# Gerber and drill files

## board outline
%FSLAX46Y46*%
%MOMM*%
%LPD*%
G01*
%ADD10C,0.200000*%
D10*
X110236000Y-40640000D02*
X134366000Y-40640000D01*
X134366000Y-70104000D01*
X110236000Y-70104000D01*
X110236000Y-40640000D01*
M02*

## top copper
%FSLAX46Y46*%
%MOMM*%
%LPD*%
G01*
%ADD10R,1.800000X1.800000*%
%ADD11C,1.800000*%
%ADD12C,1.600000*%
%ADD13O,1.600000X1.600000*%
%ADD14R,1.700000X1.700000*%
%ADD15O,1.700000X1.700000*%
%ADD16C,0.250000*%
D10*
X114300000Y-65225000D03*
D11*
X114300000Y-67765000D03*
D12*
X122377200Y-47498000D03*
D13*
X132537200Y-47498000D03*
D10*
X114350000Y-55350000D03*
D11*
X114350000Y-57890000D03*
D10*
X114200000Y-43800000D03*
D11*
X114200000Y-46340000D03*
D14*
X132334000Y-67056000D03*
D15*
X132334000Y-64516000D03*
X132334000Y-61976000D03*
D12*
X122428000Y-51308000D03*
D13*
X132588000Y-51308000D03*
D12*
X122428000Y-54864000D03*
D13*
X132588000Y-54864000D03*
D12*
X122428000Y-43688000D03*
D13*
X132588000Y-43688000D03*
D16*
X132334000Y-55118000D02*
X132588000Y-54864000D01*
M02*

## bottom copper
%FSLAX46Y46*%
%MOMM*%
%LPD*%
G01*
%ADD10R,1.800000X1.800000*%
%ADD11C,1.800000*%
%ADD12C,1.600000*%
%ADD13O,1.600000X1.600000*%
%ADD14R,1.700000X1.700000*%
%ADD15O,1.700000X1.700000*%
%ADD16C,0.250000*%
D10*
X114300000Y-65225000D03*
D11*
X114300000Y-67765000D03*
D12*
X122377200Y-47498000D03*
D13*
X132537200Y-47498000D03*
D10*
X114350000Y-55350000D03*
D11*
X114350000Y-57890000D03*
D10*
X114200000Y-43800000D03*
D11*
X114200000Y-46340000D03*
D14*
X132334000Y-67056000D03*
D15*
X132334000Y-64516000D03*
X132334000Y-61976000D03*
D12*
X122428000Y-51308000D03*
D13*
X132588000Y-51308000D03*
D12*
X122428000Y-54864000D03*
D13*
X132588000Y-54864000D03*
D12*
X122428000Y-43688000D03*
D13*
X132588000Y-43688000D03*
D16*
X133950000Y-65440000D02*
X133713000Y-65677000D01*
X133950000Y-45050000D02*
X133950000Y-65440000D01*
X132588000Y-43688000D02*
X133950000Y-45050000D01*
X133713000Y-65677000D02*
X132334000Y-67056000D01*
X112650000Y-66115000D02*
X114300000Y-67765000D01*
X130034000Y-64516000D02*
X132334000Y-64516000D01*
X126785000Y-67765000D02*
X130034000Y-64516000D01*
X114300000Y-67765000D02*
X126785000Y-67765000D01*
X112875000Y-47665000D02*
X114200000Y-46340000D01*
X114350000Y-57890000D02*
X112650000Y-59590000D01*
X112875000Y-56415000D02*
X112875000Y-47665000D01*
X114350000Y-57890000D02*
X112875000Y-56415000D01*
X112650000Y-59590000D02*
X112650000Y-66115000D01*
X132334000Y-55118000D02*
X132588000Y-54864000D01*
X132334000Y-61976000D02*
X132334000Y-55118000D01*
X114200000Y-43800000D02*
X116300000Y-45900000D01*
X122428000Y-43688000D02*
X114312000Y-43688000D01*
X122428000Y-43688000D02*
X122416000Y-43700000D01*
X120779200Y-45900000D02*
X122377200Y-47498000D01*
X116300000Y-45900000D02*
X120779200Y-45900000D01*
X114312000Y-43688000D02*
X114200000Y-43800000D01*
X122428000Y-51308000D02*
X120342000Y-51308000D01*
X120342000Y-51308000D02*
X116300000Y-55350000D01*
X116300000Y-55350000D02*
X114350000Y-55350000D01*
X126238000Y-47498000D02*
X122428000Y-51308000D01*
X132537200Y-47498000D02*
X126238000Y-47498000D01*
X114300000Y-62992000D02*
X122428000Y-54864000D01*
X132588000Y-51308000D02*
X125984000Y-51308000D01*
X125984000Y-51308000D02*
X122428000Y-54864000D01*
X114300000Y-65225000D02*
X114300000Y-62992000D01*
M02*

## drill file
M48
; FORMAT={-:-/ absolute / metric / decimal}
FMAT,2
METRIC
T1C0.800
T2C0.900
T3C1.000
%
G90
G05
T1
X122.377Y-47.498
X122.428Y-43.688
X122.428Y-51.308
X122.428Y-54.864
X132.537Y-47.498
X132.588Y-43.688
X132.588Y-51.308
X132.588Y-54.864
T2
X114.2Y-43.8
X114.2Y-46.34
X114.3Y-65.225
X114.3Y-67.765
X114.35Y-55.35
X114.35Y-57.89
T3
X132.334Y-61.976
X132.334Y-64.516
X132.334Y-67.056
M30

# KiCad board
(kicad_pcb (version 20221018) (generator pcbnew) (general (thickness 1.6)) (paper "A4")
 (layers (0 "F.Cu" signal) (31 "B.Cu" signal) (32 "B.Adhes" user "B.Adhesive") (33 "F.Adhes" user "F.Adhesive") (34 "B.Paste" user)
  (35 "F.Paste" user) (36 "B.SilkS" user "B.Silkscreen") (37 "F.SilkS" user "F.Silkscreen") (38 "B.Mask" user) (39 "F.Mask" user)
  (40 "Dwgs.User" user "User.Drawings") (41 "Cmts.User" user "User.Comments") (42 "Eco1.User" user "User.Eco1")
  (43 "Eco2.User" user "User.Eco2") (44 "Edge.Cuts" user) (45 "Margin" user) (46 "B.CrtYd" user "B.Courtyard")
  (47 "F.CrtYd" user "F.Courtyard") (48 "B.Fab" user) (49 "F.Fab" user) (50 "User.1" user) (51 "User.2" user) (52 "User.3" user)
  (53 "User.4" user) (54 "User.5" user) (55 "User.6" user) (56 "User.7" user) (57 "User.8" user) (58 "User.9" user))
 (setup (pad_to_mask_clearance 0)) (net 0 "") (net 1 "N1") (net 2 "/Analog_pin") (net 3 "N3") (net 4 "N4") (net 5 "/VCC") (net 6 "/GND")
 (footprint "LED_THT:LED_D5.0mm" (layer "F.Cu") (at 114.3 65.225 -90)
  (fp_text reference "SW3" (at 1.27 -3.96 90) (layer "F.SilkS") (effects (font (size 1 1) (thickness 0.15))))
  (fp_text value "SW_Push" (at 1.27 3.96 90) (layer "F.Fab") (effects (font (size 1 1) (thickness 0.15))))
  (pad "1" thru_hole rect (at 0 0 270) (size 1.8 1.8) (drill 0.9) (layers "*.Cu" "*.Mask") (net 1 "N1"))
  (pad "2" thru_hole circle (at 2.54 0 270) (size 1.8 1.8) (drill 0.9) (layers "*.Cu" "*.Mask") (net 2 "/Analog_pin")))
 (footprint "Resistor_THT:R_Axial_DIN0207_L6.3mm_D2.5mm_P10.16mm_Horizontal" (layer "F.Cu") (at 122.3772 47.498)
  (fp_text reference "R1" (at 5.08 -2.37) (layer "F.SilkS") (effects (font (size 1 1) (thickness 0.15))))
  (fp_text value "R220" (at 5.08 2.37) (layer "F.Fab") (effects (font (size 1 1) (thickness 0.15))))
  (pad "1" thru_hole circle (at 0 0) (size 1.6 1.6) (drill 0.8) (layers "*.Cu" "*.Mask") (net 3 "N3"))
  (pad "2" thru_hole oval (at 10.16 0) (size 1.6 1.6) (drill 0.8) (layers "*.Cu" "*.Mask") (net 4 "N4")))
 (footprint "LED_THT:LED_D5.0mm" (layer "F.Cu") (at 114.35 55.35 -90)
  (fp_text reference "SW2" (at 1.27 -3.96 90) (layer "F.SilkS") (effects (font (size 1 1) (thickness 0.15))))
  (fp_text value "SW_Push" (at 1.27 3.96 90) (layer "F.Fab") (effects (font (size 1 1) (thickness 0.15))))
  (pad "1" thru_hole rect (at 0 0 270) (size 1.8 1.8) (drill 0.9) (layers "*.Cu" "*.Mask") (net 4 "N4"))
  (pad "2" thru_hole circle (at 2.54 0 270) (size 1.8 1.8) (drill 0.9) (layers "*.Cu" "*.Mask") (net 2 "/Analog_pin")))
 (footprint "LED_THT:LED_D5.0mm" (layer "F.Cu") (at 114.2 43.8 -90)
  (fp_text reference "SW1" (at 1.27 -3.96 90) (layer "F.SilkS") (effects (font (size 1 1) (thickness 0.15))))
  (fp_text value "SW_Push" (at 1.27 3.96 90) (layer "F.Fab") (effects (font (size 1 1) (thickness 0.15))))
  (pad "1" thru_hole rect (at 0 0 270) (size 1.8 1.8) (drill 0.9) (layers "*.Cu" "*.Mask") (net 3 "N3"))
  (pad "2" thru_hole circle (at 2.54 0 270) (size 1.8 1.8) (drill 0.9) (layers "*.Cu" "*.Mask") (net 2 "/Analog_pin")))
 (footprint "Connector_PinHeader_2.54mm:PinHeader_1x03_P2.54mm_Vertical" (layer "F.Cu") (at 132.334 67.056 180)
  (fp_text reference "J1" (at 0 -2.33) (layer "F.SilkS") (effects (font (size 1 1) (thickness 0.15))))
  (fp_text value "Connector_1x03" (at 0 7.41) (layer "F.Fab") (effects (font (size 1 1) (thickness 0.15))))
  (pad "1" thru_hole rect (at 0 0 180) (size 1.7 1.7) (drill 1) (layers "*.Cu" "*.Mask") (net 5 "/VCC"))
  (pad "2" thru_hole oval (at 0 2.54 180) (size 1.7 1.7) (drill 1) (layers "*.Cu" "*.Mask") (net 2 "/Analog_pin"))
  (pad "3" thru_hole oval (at 0 5.08 180) (size 1.7 1.7) (drill 1) (layers "*.Cu" "*.Mask") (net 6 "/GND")))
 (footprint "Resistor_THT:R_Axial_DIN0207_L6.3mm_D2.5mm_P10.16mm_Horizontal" (layer "F.Cu") (at 122.428 51.308)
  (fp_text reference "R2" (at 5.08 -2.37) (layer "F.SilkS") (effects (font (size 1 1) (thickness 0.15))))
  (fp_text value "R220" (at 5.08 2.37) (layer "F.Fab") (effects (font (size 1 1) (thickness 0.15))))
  (pad "1" thru_hole circle (at 0 0) (size 1.6 1.6) (drill 0.8) (layers "*.Cu" "*.Mask") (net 4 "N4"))
  (pad "2" thru_hole oval (at 10.16 0) (size 1.6 1.6) (drill 0.8) (layers "*.Cu" "*.Mask") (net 1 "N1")))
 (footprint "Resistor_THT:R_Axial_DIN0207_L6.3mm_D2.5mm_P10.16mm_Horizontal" (layer "F.Cu") (at 122.428 54.864)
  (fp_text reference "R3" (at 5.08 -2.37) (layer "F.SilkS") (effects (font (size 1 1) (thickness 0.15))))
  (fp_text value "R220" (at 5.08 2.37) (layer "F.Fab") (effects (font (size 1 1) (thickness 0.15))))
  (pad "1" thru_hole circle (at 0 0) (size 1.6 1.6) (drill 0.8) (layers "*.Cu" "*.Mask") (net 1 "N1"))
  (pad "2" thru_hole oval (at 10.16 0) (size 1.6 1.6) (drill 0.8) (layers "*.Cu" "*.Mask") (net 6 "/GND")))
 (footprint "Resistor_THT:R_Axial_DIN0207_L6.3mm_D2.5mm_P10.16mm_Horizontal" (layer "F.Cu") (at 122.428 43.688)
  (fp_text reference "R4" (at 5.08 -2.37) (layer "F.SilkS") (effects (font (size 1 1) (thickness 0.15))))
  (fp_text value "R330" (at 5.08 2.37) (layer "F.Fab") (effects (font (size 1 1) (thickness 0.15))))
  (pad "1" thru_hole circle (at 0 0) (size 1.6 1.6) (drill 0.8) (layers "*.Cu" "*.Mask") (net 3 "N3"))
  (pad "2" thru_hole oval (at 10.16 0) (size 1.6 1.6) (drill 0.8) (layers "*.Cu" "*.Mask") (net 5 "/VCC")))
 (gr_rect (start 110.236 40.64) (end 134.366 70.104) (stroke (width 0.2) (type default)) (fill none) (layer "Edge.Cuts"))
 (segment (start 133.95 65.44) (end 133.713 65.677) (width 0.25) (layer "B.Cu") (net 5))
 (segment (start 133.95 45.05) (end 133.95 65.44) (width 0.25) (layer "B.Cu") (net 5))
 (segment (start 132.588 43.688) (end 133.95 45.05) (width 0.25) (layer "B.Cu") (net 5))
 (segment (start 133.713 65.677) (end 132.334 67.056) (width 0.25) (layer "B.Cu") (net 5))
 (segment (start 112.65 66.115) (end 114.3 67.765) (width 0.25) (layer "B.Cu") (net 2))
 (segment (start 130.034 64.516) (end 132.334 64.516) (width 0.25) (layer "B.Cu") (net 2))
 (segment (start 126.785 67.765) (end 130.034 64.516) (width 0.25) (layer "B.Cu") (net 2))
 (segment (start 114.3 67.765) (end 126.785 67.765) (width 0.25) (layer "B.Cu") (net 2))
 (segment (start 112.875 47.665) (end 114.2 46.34) (width 0.25) (layer "B.Cu") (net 2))
 (segment (start 114.35 57.89) (end 112.65 59.59) (width 0.25) (layer "B.Cu") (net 2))
 (segment (start 112.875 56.415) (end 112.875 47.665) (width 0.25) (layer "B.Cu") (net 2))
 (segment (start 114.35 57.89) (end 112.875 56.415) (width 0.25) (layer "B.Cu") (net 2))
 (segment (start 112.65 59.59) (end 112.65 66.115) (width 0.25) (layer "B.Cu") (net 2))
 (segment (start 132.334 55.118) (end 132.588 54.864) (width 0.25) (layer "F.Cu") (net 6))
 (segment (start 132.334 55.118) (end 132.588 54.864) (width 0.25) (layer "B.Cu") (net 6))
 (segment (start 132.334 61.976) (end 132.334 55.118) (width 0.25) (layer "B.Cu") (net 6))
 (segment (start 114.2 43.8) (end 116.3 45.9) (width 0.25) (layer "B.Cu") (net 3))
 (segment (start 122.428 43.688) (end 114.312 43.688) (width 0.25) (layer "B.Cu") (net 3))
 (segment (start 122.428 43.688) (end 122.416 43.7) (width 0.25) (layer "B.Cu") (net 3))
 (segment (start 120.7792 45.9) (end 122.3772 47.498) (width 0.25) (layer "B.Cu") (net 3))
 (segment (start 116.3 45.9) (end 120.7792 45.9) (width 0.25) (layer "B.Cu") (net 3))
 (segment (start 114.312 43.688) (end 114.2 43.8) (width 0.25) (layer "B.Cu") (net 3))
 (segment (start 122.428 51.308) (end 120.342 51.308) (width 0.25) (layer "B.Cu") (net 4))
 (segment (start 120.342 51.308) (end 116.3 55.35) (width 0.25) (layer "B.Cu") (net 4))
 (segment (start 116.3 55.35) (end 114.35 55.35) (width 0.25) (layer "B.Cu") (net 4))
 (segment (start 126.238 47.498) (end 122.428 51.308) (width 0.25) (layer "B.Cu") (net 4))
 (segment (start 132.5372 47.498) (end 126.238 47.498) (width 0.25) (layer "B.Cu") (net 4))
 (segment (start 114.3 62.992) (end 122.428 54.864) (width 0.25) (layer "B.Cu") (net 1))
 (segment (start 132.588 51.308) (end 125.984 51.308) (width 0.25) (layer "B.Cu") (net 1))
 (segment (start 125.984 51.308) (end 122.428 54.864) (width 0.25) (layer "B.Cu") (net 1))
 (segment (start 114.3 65.225) (end 114.3 62.992) (width 0.25) (layer "B.Cu") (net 1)))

